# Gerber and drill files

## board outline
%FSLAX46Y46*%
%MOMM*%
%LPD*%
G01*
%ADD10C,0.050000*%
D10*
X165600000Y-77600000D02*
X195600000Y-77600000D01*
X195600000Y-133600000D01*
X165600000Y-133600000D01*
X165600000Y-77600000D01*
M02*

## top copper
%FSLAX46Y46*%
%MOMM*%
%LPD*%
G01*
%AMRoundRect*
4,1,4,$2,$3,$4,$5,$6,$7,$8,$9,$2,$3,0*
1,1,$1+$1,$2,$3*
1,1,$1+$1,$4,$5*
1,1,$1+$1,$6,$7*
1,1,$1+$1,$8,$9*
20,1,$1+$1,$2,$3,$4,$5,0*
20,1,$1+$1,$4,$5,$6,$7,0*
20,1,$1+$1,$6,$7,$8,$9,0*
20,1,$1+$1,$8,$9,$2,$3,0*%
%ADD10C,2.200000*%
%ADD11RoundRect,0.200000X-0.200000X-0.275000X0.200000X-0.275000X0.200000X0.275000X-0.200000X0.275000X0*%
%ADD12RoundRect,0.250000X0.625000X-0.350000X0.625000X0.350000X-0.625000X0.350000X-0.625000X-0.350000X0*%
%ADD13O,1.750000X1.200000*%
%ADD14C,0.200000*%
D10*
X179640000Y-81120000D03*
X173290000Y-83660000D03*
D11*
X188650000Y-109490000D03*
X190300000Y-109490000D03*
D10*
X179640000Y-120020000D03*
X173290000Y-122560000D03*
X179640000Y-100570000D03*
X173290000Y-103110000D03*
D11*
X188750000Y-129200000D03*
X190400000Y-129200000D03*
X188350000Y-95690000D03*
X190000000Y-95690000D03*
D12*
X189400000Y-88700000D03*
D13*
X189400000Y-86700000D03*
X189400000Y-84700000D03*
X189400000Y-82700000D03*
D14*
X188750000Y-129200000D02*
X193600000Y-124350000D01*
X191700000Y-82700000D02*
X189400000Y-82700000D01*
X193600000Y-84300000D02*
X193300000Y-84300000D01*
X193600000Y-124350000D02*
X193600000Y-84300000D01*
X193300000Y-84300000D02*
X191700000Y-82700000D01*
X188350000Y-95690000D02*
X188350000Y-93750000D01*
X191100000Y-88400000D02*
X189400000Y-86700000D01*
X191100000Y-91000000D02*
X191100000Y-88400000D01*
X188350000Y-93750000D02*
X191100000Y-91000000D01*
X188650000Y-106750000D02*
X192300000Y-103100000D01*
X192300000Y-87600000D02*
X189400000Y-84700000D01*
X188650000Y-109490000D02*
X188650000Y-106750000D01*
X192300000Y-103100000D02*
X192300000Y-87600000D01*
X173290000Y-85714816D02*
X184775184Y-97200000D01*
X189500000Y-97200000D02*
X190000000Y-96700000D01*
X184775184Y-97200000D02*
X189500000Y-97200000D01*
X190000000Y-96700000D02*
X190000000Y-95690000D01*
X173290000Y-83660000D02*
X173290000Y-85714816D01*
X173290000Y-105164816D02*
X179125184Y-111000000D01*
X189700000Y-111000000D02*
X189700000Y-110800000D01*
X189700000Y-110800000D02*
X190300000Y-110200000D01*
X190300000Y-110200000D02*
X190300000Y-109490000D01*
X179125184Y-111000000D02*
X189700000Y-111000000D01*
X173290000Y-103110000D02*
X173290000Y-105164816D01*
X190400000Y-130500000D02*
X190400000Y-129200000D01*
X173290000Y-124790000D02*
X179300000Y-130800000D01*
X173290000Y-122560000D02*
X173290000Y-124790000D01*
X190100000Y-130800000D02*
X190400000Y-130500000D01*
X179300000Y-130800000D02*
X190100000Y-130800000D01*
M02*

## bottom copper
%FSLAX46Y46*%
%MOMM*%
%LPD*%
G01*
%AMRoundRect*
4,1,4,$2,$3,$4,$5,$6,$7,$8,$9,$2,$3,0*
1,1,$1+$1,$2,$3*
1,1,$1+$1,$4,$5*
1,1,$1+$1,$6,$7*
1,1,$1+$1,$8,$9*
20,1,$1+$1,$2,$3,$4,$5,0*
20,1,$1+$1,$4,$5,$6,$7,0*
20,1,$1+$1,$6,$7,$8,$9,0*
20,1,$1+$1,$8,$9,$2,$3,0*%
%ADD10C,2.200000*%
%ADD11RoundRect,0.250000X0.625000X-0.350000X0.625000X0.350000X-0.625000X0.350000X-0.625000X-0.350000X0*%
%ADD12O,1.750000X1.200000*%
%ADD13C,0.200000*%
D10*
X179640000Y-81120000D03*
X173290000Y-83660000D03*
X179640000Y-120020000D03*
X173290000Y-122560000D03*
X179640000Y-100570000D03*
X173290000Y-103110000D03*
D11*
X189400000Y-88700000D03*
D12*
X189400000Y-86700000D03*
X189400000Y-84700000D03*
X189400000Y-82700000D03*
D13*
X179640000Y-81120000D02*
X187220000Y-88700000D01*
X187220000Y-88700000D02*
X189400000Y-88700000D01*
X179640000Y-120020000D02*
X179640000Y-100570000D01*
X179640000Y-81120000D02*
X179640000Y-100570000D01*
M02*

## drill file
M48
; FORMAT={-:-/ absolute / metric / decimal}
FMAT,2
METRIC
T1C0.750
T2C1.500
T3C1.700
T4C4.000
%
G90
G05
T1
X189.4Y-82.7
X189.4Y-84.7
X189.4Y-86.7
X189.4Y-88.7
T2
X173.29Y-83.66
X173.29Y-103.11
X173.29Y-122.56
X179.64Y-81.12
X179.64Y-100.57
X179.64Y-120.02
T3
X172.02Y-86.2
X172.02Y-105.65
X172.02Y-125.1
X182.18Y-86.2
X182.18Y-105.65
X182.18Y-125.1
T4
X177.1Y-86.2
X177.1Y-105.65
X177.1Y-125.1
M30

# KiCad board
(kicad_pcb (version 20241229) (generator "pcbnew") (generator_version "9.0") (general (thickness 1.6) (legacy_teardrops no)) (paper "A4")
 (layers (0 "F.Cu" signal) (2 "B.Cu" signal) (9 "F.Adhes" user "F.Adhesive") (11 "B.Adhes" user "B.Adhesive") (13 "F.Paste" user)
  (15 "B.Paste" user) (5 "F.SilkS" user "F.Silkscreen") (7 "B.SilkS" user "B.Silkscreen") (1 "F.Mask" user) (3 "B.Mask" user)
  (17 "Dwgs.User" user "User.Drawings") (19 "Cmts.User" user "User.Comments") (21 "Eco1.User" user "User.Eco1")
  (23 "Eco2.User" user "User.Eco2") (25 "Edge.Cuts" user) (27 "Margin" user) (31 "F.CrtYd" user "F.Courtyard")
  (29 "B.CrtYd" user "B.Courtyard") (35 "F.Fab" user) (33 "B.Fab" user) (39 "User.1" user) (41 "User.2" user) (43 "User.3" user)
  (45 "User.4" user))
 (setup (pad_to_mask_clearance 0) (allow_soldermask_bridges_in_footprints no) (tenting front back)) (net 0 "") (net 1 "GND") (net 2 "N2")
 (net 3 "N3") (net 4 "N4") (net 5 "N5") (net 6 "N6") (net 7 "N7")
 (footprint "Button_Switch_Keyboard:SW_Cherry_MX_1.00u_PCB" (layer "F.Cu") (at 179.64 81.12)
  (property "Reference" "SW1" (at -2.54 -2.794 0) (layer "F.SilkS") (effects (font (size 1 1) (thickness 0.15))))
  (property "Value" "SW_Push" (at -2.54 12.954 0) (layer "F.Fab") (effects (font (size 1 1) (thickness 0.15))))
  (pad "" np_thru_hole circle (at -7.62 5.08) (size 1.7 1.7) (drill 1.7) (layers "*.Cu" "*.Mask"))
  (pad "" np_thru_hole circle (at -2.54 5.08) (size 4 4) (drill 4) (layers "*.Cu" "*.Mask"))
  (pad "" np_thru_hole circle (at 2.54 5.08) (size 1.7 1.7) (drill 1.7) (layers "*.Cu" "*.Mask"))
  (pad "1" thru_hole circle (at 0 0) (size 2.2 2.2) (drill 1.5) (layers "*.Cu" "*.Mask") (remove_unused_layers no) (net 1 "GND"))
  (pad "2" thru_hole circle (at -6.35 2.54) (size 2.2 2.2) (drill 1.5) (layers "*.Cu" "*.Mask") (remove_unused_layers no) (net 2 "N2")))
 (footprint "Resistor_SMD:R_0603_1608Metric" (layer "F.Cu") (at 189.475 109.49)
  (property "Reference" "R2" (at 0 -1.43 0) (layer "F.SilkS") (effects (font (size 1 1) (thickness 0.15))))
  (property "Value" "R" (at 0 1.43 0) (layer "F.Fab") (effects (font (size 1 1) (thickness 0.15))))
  (pad "1" smd roundrect (at -0.825 0) (size 0.8 0.95) (layers "F.Cu" "F.Mask" "F.Paste") (roundrect_rratio 0.25) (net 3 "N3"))
  (pad "2" smd roundrect (at 0.825 0) (size 0.8 0.95) (layers "F.Cu" "F.Mask" "F.Paste") (roundrect_rratio 0.25) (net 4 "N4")))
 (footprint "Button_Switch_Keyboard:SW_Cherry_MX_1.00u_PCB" (layer "F.Cu") (at 179.64 120.02)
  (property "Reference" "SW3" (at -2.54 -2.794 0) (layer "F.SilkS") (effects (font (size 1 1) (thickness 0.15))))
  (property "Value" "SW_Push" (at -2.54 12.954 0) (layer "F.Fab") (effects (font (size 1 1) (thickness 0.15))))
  (pad "" np_thru_hole circle (at -7.62 5.08) (size 1.7 1.7) (drill 1.7) (layers "*.Cu" "*.Mask"))
  (pad "" np_thru_hole circle (at -2.54 5.08) (size 4 4) (drill 4) (layers "*.Cu" "*.Mask"))
  (pad "" np_thru_hole circle (at 2.54 5.08) (size 1.7 1.7) (drill 1.7) (layers "*.Cu" "*.Mask"))
  (pad "1" thru_hole circle (at 0 0) (size 2.2 2.2) (drill 1.5) (layers "*.Cu" "*.Mask") (remove_unused_layers no) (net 1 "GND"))
  (pad "2" thru_hole circle (at -6.35 2.54) (size 2.2 2.2) (drill 1.5) (layers "*.Cu" "*.Mask") (remove_unused_layers no) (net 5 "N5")))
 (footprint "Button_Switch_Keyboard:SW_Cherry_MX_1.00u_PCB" (layer "F.Cu") (at 179.64 100.57)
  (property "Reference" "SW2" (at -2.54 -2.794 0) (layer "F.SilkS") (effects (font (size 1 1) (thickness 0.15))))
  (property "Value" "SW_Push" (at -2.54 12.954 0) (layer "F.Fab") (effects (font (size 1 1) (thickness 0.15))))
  (pad "" np_thru_hole circle (at -7.62 5.08) (size 1.7 1.7) (drill 1.7) (layers "*.Cu" "*.Mask"))
  (pad "" np_thru_hole circle (at -2.54 5.08) (size 4 4) (drill 4) (layers "*.Cu" "*.Mask"))
  (pad "" np_thru_hole circle (at 2.54 5.08) (size 1.7 1.7) (drill 1.7) (layers "*.Cu" "*.Mask"))
  (pad "1" thru_hole circle (at 0 0) (size 2.2 2.2) (drill 1.5) (layers "*.Cu" "*.Mask") (remove_unused_layers no) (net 1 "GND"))
  (pad "2" thru_hole circle (at -6.35 2.54) (size 2.2 2.2) (drill 1.5) (layers "*.Cu" "*.Mask") (remove_unused_layers no) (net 4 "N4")))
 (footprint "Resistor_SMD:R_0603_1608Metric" (layer "F.Cu") (at 189.575 129.2)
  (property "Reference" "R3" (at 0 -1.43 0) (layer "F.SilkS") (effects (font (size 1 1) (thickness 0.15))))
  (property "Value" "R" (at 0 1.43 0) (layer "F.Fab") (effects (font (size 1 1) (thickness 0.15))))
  (pad "1" smd roundrect (at -0.825 0) (size 0.8 0.95) (layers "F.Cu" "F.Mask" "F.Paste") (roundrect_rratio 0.25) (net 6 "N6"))
  (pad "2" smd roundrect (at 0.825 0) (size 0.8 0.95) (layers "F.Cu" "F.Mask" "F.Paste") (roundrect_rratio 0.25) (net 5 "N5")))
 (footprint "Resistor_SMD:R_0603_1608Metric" (layer "F.Cu") (at 189.175 95.69)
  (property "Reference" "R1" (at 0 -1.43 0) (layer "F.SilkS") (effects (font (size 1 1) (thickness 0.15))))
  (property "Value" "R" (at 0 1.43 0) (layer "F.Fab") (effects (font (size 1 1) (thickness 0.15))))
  (pad "1" smd roundrect (at -0.825 0) (size 0.8 0.95) (layers "F.Cu" "F.Mask" "F.Paste") (roundrect_rratio 0.25) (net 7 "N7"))
  (pad "2" smd roundrect (at 0.825 0) (size 0.8 0.95) (layers "F.Cu" "F.Mask" "F.Paste") (roundrect_rratio 0.25) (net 2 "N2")))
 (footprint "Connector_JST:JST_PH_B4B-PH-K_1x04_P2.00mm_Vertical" (layer "F.Cu") (at 189.4 88.7 90)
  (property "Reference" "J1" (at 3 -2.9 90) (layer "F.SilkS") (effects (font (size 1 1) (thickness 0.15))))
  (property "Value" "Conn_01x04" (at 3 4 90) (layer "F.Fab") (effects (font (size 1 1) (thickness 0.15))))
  (pad "1" thru_hole roundrect (at 0 0 90) (size 1.2 1.75) (drill 0.75) (layers "*.Cu" "*.Mask") (remove_unused_layers no)
   (roundrect_rratio 0.208333) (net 1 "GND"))
  (pad "2" thru_hole oval (at 2 0 90) (size 1.2 1.75) (drill 0.75) (layers "*.Cu" "*.Mask") (remove_unused_layers no) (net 7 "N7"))
  (pad "3" thru_hole oval (at 4 0 90) (size 1.2 1.75) (drill 0.75) (layers "*.Cu" "*.Mask") (remove_unused_layers no) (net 3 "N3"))
  (pad "4" thru_hole oval (at 6 0 90) (size 1.2 1.75) (drill 0.75) (layers "*.Cu" "*.Mask") (remove_unused_layers no) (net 6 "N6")))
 (gr_rect (start 165.6 77.6) (end 195.6 133.6) (stroke (width 0.05) (type default)) (fill no) (layer "Edge.Cuts"))
 (segment (start 188.75 129.2) (end 193.6 124.35) (width 0.2) (layer "F.Cu") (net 6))
 (segment (start 191.7 82.7) (end 189.4 82.7) (width 0.2) (layer "F.Cu") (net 6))
 (segment (start 193.6 84.3) (end 193.3 84.3) (width 0.2) (layer "F.Cu") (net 6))
 (segment (start 193.6 124.35) (end 193.6 84.3) (width 0.2) (layer "F.Cu") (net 6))
 (segment (start 193.3 84.3) (end 191.7 82.7) (width 0.2) (layer "F.Cu") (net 6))
 (segment (start 179.64 81.12) (end 187.22 88.7) (width 0.2) (layer "B.Cu") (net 1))
 (segment (start 187.22 88.7) (end 189.4 88.7) (width 0.2) (layer "B.Cu") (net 1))
 (segment (start 179.64 120.02) (end 179.64 100.57) (width 0.2) (layer "B.Cu") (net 1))
 (segment (start 179.64 81.12) (end 179.64 100.57) (width 0.2) (layer "B.Cu") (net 1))
 (segment (start 188.35 95.69) (end 188.35 93.75) (width 0.2) (layer "F.Cu") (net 7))
 (segment (start 191.1 88.4) (end 189.4 86.7) (width 0.2) (layer "F.Cu") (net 7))
 (segment (start 191.1 91) (end 191.1 88.4) (width 0.2) (layer "F.Cu") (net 7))
 (segment (start 188.35 93.75) (end 191.1 91) (width 0.2) (layer "F.Cu") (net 7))
 (segment (start 188.65 106.75) (end 192.3 103.1) (width 0.2) (layer "F.Cu") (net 3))
 (segment (start 192.3 87.6) (end 189.4 84.7) (width 0.2) (layer "F.Cu") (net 3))
 (segment (start 188.65 109.49) (end 188.65 106.75) (width 0.2) (layer "F.Cu") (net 3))
 (segment (start 192.3 103.1) (end 192.3 87.6) (width 0.2) (layer "F.Cu") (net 3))
 (segment (start 173.29 85.714816) (end 184.775184 97.2) (width 0.2) (layer "F.Cu") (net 2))
 (segment (start 189.5 97.2) (end 190 96.7) (width 0.2) (layer "F.Cu") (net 2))
 (segment (start 184.775184 97.2) (end 189.5 97.2) (width 0.2) (layer "F.Cu") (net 2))
 (segment (start 190 96.7) (end 190 95.69) (width 0.2) (layer "F.Cu") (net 2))
 (segment (start 173.29 83.66) (end 173.29 85.714816) (width 0.2) (layer "F.Cu") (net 2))
 (segment (start 173.29 105.164816) (end 179.125184 111) (width 0.2) (layer "F.Cu") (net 4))
 (segment (start 189.7 111) (end 189.7 110.8) (width 0.2) (layer "F.Cu") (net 4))
 (segment (start 189.7 110.8) (end 190.3 110.2) (width 0.2) (layer "F.Cu") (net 4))
 (segment (start 190.3 110.2) (end 190.3 109.49) (width 0.2) (layer "F.Cu") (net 4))
 (segment (start 179.125184 111) (end 189.7 111) (width 0.2) (layer "F.Cu") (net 4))
 (segment (start 173.29 103.11) (end 173.29 105.164816) (width 0.2) (layer "F.Cu") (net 4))
 (segment (start 190.4 130.5) (end 190.4 129.2) (width 0.2) (layer "F.Cu") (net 5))
 (segment (start 173.29 124.79) (end 179.3 130.8) (width 0.2) (layer "F.Cu") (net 5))
 (segment (start 173.29 122.56) (end 173.29 124.79) (width 0.2) (layer "F.Cu") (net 5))
 (segment (start 190.1 130.8) (end 190.4 130.5) (width 0.2) (layer "F.Cu") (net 5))
 (segment (start 179.3 130.8) (end 190.1 130.8) (width 0.2) (layer "F.Cu") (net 5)))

